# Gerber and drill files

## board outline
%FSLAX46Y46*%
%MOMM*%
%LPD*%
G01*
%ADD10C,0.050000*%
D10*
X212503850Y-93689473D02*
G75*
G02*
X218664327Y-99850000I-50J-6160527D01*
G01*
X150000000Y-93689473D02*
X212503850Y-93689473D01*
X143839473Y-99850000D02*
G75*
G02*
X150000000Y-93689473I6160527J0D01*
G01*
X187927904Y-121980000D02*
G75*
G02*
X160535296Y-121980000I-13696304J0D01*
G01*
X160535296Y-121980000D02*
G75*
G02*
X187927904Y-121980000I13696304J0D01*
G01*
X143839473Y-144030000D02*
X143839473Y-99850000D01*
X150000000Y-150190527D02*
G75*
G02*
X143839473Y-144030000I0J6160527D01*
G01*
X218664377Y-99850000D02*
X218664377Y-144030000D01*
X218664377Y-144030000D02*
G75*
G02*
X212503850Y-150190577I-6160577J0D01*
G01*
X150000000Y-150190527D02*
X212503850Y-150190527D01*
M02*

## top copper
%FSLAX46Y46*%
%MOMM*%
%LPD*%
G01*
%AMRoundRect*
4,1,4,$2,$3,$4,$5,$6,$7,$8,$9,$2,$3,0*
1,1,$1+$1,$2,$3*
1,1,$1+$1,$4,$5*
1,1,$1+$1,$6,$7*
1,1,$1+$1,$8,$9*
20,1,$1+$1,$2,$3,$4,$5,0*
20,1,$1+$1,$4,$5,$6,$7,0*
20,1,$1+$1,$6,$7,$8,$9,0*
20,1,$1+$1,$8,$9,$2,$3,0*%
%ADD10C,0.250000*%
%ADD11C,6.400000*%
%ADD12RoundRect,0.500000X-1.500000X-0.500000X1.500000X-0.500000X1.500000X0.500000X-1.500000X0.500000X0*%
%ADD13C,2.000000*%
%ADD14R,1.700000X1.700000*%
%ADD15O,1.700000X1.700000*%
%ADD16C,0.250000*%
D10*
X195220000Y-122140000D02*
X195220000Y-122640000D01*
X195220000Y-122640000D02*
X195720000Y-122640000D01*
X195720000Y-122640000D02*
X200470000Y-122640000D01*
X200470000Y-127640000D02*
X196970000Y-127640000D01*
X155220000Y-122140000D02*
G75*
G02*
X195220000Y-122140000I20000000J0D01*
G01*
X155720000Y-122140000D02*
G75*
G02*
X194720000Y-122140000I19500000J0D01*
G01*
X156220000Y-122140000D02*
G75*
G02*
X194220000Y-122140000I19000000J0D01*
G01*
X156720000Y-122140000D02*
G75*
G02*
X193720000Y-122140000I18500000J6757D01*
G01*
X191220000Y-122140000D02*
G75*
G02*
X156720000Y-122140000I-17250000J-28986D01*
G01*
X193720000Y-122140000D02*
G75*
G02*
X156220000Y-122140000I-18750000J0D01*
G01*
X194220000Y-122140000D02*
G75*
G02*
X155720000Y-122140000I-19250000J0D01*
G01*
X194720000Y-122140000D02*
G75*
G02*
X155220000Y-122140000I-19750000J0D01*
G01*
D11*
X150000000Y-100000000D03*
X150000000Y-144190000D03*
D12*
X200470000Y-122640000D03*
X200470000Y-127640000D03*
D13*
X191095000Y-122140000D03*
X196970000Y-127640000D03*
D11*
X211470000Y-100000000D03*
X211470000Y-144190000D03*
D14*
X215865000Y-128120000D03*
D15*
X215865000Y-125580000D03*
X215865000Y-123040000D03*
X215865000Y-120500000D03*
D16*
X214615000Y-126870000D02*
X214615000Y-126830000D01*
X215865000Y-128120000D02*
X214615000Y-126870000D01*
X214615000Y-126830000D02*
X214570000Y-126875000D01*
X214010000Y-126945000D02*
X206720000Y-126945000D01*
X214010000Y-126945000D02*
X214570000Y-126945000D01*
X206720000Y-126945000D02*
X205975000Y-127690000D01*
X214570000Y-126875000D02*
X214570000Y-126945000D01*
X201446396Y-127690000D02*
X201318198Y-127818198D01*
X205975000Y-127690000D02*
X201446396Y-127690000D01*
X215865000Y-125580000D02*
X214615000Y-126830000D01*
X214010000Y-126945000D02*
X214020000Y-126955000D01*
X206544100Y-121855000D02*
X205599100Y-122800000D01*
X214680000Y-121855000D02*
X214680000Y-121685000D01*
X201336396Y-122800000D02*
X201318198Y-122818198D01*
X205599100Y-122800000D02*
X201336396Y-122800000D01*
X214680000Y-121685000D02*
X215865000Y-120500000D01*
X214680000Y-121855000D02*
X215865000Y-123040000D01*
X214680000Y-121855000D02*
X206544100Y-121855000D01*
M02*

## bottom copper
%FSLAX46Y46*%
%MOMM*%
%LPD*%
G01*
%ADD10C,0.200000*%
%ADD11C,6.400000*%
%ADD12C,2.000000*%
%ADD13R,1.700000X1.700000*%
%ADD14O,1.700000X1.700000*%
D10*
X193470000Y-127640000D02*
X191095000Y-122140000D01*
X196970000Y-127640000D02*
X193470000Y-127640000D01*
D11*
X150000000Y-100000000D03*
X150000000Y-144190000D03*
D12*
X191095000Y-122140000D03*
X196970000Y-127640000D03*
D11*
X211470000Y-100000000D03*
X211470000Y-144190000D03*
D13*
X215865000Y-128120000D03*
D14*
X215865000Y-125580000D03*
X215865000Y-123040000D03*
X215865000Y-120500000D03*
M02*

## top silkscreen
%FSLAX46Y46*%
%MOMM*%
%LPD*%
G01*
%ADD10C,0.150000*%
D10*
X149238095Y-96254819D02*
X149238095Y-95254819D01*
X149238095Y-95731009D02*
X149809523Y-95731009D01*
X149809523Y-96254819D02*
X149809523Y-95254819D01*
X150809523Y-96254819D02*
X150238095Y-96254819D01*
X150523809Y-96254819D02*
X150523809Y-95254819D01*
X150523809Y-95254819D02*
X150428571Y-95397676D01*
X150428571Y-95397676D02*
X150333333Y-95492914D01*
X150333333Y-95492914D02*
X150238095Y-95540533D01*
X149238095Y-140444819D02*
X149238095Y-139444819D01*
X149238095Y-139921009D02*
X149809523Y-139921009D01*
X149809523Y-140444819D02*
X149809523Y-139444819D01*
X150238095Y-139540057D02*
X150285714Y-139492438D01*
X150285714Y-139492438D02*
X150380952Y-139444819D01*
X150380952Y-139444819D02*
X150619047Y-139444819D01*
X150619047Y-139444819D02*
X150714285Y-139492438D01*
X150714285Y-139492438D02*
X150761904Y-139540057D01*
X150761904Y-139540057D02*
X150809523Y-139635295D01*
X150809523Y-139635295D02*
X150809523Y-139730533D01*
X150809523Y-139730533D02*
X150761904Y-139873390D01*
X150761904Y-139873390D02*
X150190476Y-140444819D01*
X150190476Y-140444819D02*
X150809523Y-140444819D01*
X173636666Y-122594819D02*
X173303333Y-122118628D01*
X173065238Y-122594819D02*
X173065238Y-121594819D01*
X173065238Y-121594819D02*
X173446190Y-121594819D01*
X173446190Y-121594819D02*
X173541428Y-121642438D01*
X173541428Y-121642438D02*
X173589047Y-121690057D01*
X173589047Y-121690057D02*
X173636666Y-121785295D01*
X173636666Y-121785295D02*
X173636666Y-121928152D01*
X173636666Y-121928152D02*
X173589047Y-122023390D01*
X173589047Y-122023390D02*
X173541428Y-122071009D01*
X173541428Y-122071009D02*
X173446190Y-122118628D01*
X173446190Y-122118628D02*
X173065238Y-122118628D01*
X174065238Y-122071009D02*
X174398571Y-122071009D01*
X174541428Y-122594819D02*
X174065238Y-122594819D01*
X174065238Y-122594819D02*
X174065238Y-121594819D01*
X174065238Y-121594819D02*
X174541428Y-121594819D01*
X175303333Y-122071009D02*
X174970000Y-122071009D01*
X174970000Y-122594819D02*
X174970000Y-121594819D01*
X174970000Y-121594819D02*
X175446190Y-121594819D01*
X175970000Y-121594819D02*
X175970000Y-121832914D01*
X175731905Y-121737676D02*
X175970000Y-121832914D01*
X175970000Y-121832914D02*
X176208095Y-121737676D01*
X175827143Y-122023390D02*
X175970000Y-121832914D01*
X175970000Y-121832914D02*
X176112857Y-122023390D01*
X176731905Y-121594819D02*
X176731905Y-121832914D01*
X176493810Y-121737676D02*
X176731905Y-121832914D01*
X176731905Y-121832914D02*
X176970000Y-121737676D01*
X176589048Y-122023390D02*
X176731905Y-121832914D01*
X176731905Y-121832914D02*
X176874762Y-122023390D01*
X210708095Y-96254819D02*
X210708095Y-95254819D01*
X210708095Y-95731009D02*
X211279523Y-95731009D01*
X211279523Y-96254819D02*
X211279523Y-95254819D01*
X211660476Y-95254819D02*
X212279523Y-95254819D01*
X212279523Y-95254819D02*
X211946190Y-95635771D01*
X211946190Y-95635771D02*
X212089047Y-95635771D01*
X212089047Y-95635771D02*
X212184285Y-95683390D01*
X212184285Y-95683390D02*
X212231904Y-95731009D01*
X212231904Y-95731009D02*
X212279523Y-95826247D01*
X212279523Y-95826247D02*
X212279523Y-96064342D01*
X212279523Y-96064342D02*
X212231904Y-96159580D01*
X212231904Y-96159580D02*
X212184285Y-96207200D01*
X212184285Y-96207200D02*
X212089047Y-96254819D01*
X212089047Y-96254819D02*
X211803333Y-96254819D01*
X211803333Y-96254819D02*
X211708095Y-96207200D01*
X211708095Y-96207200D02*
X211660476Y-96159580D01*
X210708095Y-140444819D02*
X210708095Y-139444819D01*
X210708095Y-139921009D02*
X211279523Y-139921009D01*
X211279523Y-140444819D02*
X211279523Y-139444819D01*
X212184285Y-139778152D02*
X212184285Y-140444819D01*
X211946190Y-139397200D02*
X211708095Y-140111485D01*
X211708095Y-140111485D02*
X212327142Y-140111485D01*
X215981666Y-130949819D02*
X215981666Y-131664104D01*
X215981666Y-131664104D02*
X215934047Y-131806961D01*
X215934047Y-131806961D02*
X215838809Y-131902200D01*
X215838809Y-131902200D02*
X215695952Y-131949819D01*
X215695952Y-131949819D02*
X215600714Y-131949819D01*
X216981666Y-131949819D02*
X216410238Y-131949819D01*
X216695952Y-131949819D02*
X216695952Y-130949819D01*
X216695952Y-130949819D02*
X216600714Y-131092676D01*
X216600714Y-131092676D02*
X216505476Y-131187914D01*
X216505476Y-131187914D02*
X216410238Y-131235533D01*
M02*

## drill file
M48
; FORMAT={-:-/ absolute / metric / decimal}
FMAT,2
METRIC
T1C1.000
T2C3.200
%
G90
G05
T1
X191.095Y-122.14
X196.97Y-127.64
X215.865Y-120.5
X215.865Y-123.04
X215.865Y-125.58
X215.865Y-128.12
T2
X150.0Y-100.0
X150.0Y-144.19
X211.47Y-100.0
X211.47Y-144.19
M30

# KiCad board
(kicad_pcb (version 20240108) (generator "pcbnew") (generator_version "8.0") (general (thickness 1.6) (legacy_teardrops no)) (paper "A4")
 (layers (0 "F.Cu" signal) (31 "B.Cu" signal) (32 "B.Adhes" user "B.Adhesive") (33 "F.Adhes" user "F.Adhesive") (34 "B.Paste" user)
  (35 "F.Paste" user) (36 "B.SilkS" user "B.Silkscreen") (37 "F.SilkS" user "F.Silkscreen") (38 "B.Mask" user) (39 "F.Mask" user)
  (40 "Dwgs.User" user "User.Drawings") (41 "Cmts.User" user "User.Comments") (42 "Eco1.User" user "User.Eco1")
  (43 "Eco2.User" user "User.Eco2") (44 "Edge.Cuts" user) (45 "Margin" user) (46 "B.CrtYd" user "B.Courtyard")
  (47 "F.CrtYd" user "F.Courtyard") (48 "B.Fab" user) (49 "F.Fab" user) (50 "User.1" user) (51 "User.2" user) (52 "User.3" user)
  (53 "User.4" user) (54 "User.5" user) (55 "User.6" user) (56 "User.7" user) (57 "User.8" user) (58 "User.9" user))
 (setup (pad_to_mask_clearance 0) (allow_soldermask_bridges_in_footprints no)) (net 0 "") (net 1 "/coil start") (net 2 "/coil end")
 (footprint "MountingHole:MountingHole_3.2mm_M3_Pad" (layer "F.Cu") (at 150 100)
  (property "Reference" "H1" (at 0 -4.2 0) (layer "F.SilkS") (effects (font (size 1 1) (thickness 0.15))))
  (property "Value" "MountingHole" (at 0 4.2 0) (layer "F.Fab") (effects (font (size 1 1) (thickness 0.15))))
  (pad "1" thru_hole circle (at 0 0) (size 6.4 6.4) (drill 3.2) (layers "*.Cu" "*.Mask") (remove_unused_layers no)))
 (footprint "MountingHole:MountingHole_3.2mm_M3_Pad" (layer "F.Cu") (at 150 144.19)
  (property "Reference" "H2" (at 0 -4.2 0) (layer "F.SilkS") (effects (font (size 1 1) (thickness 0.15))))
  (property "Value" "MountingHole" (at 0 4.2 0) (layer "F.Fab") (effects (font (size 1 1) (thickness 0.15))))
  (pad "1" thru_hole circle (at 0 0) (size 6.4 6.4) (drill 3.2) (layers "*.Cu" "*.Mask") (remove_unused_layers no)))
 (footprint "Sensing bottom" (layer "F.Cu") (at 174.97 122.14)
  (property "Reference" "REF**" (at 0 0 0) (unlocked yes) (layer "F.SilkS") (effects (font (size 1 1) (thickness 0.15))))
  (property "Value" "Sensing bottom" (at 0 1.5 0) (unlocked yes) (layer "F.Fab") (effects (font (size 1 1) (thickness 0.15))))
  (fp_line (start 20.25 0) (end 20.25 0.5) (stroke (width 0.25) (type solid)) (layer "F.Cu"))
  (fp_line (start 20.25 0.5) (end 20.75 0.5) (stroke (width 0.25) (type solid)) (layer "F.Cu"))
  (fp_line (start 20.75 0.5) (end 25.5 0.5) (stroke (width 0.25) (type default)) (layer "F.Cu"))
  (fp_line (start 25.5 5.5) (end 22 5.5) (stroke (width 0.25) (type default)) (layer "F.Cu"))
  (fp_arc (start -19.75 0) (mid 0.25 -20) (end 20.25 0) (stroke (width 0.25) (type solid)) (layer "F.Cu"))
  (fp_arc (start -19.25 0) (mid 0.25 -19.5) (end 19.75 0) (stroke (width 0.25) (type solid)) (layer "F.Cu"))
  (fp_arc (start -18.75 0) (mid 0.25 -19) (end 19.25 0) (stroke (width 0.25) (type solid)) (layer "F.Cu"))
  (fp_arc (start -18.25 0) (mid 0.25 -18.506758) (end 18.75 0) (stroke (width 0.25) (type solid)) (layer "F.Cu"))
  (fp_arc (start 16.25 0) (mid -1 17.27901) (end -18.25 0) (stroke (width 0.25) (type solid)) (layer "F.Cu"))
  (fp_arc (start 18.75 0) (mid 0 18.75) (end -18.75 0) (stroke (width 0.25) (type solid)) (layer "F.Cu"))
  (fp_arc (start 19.25 0) (mid 0 19.25) (end -19.25 0) (stroke (width 0.25) (type solid)) (layer "F.Cu"))
  (fp_arc (start 19.75 0) (mid 0 19.75) (end -19.75 0) (stroke (width 0.25) (type solid)) (layer "F.Cu"))
  (fp_line (start 18.5 5.5) (end 16.125 0) (stroke (width 0.2) (type default)) (layer "B.Cu"))
  (fp_line (start 22 5.5) (end 18.5 5.5) (stroke (width 0.2) (type default)) (layer "B.Cu"))
  (pad "1" smd roundrect (at 25.5 0.5) (size 4 2) (layers "F.Cu") (roundrect_rratio 0.25) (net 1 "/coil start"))
  (pad "2" smd roundrect (at 25.5 5.5) (size 4 2) (layers "F.Cu") (roundrect_rratio 0.25) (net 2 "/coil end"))
  (pad "3" thru_hole circle (at 16.125 0) (size 2 2) (drill 1) (layers "*.Cu" "*.Mask") (remove_unused_layers no))
  (pad "3" thru_hole circle (at 22 5.5) (size 2 2) (drill 1) (layers "*.Cu" "*.Mask") (remove_unused_layers no)))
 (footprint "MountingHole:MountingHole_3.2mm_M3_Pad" (layer "F.Cu") (at 211.47 100)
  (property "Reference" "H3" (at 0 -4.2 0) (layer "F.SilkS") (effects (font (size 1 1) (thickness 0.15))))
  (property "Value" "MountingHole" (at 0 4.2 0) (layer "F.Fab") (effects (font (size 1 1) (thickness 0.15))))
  (pad "1" thru_hole circle (at 0 0) (size 6.4 6.4) (drill 3.2) (layers "*.Cu" "*.Mask") (remove_unused_layers no)))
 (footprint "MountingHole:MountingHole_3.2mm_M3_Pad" (layer "F.Cu") (at 211.47 144.19)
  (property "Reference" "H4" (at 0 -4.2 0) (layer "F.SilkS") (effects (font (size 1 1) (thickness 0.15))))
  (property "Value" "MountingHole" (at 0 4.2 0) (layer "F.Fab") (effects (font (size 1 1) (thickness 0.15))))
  (pad "1" thru_hole circle (at 0 0) (size 6.4 6.4) (drill 3.2) (layers "*.Cu" "*.Mask") (remove_unused_layers no)))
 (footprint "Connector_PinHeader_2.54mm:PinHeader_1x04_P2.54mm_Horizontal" (layer "B.Cu") (at 215.865 128.12)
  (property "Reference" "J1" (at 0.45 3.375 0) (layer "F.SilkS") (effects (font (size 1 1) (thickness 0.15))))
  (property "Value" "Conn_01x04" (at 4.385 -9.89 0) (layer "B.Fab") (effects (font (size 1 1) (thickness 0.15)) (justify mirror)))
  (pad "1" thru_hole rect (at 0 0) (size 1.7 1.7) (drill 1) (layers "*.Cu" "*.Mask") (remove_unused_layers no) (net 2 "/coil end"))
  (pad "2" thru_hole oval (at 0 -2.54) (size 1.7 1.7) (drill 1) (layers "*.Cu" "*.Mask") (remove_unused_layers no) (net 2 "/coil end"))
  (pad "3" thru_hole oval (at 0 -5.08) (size 1.7 1.7) (drill 1) (layers "*.Cu" "*.Mask") (remove_unused_layers no) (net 1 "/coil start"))
  (pad "4" thru_hole oval (at 0 -7.62) (size 1.7 1.7) (drill 1) (layers "*.Cu" "*.Mask") (remove_unused_layers no) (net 1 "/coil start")))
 (gr_arc (start 212.50385 93.689473) (mid 216.86 95.49385) (end 218.664377 99.85) (stroke (width 0.05) (type default)) (layer "Edge.Cuts"))
 (gr_line (start 150 93.689473) (end 212.50385 93.689473) (stroke (width 0.05) (type default)) (layer "Edge.Cuts"))
 (gr_arc (start 143.839473 99.85) (mid 145.64385 95.49385) (end 150 93.689473) (stroke (width 0.05) (type default)) (layer "Edge.Cuts"))
 (gr_circle (center 174.2316 121.98) (end 186.47 115.830992) (stroke (width 0.05) (type default)) (fill none) (layer "Edge.Cuts"))
 (gr_line (start 143.839473 144.03) (end 143.839473 99.85) (stroke (width 0.05) (type default)) (layer "Edge.Cuts"))
 (gr_arc (start 150 150.190527) (mid 145.643849 148.38615) (end 143.839473 144.03) (stroke (width 0.05) (type default)) (layer "Edge.Cuts"))
 (gr_line (start 218.664377 99.85) (end 218.664377 144.03) (stroke (width 0.05) (type default)) (layer "Edge.Cuts"))
 (gr_arc (start 218.664377 144.03) (mid 216.86 148.38615) (end 212.50385 150.190527) (stroke (width 0.05) (type default))
  (layer "Edge.Cuts"))
 (gr_line (start 150 150.190527) (end 212.50385 150.190527) (stroke (width 0.05) (type default)) (layer "Edge.Cuts"))
 (segment (start 214.615 126.87) (end 214.615 126.83) (width 0.25) (layer "F.Cu") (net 2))
 (segment (start 215.865 128.12) (end 214.615 126.87) (width 0.25) (layer "F.Cu") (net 2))
 (segment (start 214.615 126.83) (end 214.57 126.875) (width 0.25) (layer "F.Cu") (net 2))
 (segment (start 214.01 126.945) (end 206.72 126.945) (width 0.25) (layer "F.Cu") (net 2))
 (segment (start 214.01 126.945) (end 214.57 126.945) (width 0.25) (layer "F.Cu") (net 2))
 (segment (start 206.72 126.945) (end 205.975 127.69) (width 0.25) (layer "F.Cu") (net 2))
 (segment (start 214.57 126.875) (end 214.57 126.945) (width 0.25) (layer "F.Cu") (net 2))
 (segment (start 201.446396 127.69) (end 201.318198 127.818198) (width 0.25) (layer "F.Cu") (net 2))
 (segment (start 205.975 127.69) (end 201.446396 127.69) (width 0.25) (layer "F.Cu") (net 2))
 (segment (start 215.865 125.58) (end 214.615 126.83) (width 0.25) (layer "F.Cu") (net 2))
 (segment (start 214.01 126.945) (end 214.02 126.955) (width 0.25) (layer "F.Cu") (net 2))
 (segment (start 206.5441 121.855) (end 205.5991 122.8) (width 0.25) (layer "F.Cu") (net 1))
 (segment (start 214.68 121.855) (end 214.68 121.685) (width 0.25) (layer "F.Cu") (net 1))
 (segment (start 201.336396 122.8) (end 201.318198 122.818198) (width 0.25) (layer "F.Cu") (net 1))
 (segment (start 205.5991 122.8) (end 201.336396 122.8) (width 0.25) (layer "F.Cu") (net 1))
 (segment (start 214.68 121.685) (end 215.865 120.5) (width 0.25) (layer "F.Cu") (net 1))
 (segment (start 214.68 121.855) (end 215.865 123.04) (width 0.25) (layer "F.Cu") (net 1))
 (segment (start 214.68 121.855) (end 206.5441 121.855) (width 0.25) (layer "F.Cu") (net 1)))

